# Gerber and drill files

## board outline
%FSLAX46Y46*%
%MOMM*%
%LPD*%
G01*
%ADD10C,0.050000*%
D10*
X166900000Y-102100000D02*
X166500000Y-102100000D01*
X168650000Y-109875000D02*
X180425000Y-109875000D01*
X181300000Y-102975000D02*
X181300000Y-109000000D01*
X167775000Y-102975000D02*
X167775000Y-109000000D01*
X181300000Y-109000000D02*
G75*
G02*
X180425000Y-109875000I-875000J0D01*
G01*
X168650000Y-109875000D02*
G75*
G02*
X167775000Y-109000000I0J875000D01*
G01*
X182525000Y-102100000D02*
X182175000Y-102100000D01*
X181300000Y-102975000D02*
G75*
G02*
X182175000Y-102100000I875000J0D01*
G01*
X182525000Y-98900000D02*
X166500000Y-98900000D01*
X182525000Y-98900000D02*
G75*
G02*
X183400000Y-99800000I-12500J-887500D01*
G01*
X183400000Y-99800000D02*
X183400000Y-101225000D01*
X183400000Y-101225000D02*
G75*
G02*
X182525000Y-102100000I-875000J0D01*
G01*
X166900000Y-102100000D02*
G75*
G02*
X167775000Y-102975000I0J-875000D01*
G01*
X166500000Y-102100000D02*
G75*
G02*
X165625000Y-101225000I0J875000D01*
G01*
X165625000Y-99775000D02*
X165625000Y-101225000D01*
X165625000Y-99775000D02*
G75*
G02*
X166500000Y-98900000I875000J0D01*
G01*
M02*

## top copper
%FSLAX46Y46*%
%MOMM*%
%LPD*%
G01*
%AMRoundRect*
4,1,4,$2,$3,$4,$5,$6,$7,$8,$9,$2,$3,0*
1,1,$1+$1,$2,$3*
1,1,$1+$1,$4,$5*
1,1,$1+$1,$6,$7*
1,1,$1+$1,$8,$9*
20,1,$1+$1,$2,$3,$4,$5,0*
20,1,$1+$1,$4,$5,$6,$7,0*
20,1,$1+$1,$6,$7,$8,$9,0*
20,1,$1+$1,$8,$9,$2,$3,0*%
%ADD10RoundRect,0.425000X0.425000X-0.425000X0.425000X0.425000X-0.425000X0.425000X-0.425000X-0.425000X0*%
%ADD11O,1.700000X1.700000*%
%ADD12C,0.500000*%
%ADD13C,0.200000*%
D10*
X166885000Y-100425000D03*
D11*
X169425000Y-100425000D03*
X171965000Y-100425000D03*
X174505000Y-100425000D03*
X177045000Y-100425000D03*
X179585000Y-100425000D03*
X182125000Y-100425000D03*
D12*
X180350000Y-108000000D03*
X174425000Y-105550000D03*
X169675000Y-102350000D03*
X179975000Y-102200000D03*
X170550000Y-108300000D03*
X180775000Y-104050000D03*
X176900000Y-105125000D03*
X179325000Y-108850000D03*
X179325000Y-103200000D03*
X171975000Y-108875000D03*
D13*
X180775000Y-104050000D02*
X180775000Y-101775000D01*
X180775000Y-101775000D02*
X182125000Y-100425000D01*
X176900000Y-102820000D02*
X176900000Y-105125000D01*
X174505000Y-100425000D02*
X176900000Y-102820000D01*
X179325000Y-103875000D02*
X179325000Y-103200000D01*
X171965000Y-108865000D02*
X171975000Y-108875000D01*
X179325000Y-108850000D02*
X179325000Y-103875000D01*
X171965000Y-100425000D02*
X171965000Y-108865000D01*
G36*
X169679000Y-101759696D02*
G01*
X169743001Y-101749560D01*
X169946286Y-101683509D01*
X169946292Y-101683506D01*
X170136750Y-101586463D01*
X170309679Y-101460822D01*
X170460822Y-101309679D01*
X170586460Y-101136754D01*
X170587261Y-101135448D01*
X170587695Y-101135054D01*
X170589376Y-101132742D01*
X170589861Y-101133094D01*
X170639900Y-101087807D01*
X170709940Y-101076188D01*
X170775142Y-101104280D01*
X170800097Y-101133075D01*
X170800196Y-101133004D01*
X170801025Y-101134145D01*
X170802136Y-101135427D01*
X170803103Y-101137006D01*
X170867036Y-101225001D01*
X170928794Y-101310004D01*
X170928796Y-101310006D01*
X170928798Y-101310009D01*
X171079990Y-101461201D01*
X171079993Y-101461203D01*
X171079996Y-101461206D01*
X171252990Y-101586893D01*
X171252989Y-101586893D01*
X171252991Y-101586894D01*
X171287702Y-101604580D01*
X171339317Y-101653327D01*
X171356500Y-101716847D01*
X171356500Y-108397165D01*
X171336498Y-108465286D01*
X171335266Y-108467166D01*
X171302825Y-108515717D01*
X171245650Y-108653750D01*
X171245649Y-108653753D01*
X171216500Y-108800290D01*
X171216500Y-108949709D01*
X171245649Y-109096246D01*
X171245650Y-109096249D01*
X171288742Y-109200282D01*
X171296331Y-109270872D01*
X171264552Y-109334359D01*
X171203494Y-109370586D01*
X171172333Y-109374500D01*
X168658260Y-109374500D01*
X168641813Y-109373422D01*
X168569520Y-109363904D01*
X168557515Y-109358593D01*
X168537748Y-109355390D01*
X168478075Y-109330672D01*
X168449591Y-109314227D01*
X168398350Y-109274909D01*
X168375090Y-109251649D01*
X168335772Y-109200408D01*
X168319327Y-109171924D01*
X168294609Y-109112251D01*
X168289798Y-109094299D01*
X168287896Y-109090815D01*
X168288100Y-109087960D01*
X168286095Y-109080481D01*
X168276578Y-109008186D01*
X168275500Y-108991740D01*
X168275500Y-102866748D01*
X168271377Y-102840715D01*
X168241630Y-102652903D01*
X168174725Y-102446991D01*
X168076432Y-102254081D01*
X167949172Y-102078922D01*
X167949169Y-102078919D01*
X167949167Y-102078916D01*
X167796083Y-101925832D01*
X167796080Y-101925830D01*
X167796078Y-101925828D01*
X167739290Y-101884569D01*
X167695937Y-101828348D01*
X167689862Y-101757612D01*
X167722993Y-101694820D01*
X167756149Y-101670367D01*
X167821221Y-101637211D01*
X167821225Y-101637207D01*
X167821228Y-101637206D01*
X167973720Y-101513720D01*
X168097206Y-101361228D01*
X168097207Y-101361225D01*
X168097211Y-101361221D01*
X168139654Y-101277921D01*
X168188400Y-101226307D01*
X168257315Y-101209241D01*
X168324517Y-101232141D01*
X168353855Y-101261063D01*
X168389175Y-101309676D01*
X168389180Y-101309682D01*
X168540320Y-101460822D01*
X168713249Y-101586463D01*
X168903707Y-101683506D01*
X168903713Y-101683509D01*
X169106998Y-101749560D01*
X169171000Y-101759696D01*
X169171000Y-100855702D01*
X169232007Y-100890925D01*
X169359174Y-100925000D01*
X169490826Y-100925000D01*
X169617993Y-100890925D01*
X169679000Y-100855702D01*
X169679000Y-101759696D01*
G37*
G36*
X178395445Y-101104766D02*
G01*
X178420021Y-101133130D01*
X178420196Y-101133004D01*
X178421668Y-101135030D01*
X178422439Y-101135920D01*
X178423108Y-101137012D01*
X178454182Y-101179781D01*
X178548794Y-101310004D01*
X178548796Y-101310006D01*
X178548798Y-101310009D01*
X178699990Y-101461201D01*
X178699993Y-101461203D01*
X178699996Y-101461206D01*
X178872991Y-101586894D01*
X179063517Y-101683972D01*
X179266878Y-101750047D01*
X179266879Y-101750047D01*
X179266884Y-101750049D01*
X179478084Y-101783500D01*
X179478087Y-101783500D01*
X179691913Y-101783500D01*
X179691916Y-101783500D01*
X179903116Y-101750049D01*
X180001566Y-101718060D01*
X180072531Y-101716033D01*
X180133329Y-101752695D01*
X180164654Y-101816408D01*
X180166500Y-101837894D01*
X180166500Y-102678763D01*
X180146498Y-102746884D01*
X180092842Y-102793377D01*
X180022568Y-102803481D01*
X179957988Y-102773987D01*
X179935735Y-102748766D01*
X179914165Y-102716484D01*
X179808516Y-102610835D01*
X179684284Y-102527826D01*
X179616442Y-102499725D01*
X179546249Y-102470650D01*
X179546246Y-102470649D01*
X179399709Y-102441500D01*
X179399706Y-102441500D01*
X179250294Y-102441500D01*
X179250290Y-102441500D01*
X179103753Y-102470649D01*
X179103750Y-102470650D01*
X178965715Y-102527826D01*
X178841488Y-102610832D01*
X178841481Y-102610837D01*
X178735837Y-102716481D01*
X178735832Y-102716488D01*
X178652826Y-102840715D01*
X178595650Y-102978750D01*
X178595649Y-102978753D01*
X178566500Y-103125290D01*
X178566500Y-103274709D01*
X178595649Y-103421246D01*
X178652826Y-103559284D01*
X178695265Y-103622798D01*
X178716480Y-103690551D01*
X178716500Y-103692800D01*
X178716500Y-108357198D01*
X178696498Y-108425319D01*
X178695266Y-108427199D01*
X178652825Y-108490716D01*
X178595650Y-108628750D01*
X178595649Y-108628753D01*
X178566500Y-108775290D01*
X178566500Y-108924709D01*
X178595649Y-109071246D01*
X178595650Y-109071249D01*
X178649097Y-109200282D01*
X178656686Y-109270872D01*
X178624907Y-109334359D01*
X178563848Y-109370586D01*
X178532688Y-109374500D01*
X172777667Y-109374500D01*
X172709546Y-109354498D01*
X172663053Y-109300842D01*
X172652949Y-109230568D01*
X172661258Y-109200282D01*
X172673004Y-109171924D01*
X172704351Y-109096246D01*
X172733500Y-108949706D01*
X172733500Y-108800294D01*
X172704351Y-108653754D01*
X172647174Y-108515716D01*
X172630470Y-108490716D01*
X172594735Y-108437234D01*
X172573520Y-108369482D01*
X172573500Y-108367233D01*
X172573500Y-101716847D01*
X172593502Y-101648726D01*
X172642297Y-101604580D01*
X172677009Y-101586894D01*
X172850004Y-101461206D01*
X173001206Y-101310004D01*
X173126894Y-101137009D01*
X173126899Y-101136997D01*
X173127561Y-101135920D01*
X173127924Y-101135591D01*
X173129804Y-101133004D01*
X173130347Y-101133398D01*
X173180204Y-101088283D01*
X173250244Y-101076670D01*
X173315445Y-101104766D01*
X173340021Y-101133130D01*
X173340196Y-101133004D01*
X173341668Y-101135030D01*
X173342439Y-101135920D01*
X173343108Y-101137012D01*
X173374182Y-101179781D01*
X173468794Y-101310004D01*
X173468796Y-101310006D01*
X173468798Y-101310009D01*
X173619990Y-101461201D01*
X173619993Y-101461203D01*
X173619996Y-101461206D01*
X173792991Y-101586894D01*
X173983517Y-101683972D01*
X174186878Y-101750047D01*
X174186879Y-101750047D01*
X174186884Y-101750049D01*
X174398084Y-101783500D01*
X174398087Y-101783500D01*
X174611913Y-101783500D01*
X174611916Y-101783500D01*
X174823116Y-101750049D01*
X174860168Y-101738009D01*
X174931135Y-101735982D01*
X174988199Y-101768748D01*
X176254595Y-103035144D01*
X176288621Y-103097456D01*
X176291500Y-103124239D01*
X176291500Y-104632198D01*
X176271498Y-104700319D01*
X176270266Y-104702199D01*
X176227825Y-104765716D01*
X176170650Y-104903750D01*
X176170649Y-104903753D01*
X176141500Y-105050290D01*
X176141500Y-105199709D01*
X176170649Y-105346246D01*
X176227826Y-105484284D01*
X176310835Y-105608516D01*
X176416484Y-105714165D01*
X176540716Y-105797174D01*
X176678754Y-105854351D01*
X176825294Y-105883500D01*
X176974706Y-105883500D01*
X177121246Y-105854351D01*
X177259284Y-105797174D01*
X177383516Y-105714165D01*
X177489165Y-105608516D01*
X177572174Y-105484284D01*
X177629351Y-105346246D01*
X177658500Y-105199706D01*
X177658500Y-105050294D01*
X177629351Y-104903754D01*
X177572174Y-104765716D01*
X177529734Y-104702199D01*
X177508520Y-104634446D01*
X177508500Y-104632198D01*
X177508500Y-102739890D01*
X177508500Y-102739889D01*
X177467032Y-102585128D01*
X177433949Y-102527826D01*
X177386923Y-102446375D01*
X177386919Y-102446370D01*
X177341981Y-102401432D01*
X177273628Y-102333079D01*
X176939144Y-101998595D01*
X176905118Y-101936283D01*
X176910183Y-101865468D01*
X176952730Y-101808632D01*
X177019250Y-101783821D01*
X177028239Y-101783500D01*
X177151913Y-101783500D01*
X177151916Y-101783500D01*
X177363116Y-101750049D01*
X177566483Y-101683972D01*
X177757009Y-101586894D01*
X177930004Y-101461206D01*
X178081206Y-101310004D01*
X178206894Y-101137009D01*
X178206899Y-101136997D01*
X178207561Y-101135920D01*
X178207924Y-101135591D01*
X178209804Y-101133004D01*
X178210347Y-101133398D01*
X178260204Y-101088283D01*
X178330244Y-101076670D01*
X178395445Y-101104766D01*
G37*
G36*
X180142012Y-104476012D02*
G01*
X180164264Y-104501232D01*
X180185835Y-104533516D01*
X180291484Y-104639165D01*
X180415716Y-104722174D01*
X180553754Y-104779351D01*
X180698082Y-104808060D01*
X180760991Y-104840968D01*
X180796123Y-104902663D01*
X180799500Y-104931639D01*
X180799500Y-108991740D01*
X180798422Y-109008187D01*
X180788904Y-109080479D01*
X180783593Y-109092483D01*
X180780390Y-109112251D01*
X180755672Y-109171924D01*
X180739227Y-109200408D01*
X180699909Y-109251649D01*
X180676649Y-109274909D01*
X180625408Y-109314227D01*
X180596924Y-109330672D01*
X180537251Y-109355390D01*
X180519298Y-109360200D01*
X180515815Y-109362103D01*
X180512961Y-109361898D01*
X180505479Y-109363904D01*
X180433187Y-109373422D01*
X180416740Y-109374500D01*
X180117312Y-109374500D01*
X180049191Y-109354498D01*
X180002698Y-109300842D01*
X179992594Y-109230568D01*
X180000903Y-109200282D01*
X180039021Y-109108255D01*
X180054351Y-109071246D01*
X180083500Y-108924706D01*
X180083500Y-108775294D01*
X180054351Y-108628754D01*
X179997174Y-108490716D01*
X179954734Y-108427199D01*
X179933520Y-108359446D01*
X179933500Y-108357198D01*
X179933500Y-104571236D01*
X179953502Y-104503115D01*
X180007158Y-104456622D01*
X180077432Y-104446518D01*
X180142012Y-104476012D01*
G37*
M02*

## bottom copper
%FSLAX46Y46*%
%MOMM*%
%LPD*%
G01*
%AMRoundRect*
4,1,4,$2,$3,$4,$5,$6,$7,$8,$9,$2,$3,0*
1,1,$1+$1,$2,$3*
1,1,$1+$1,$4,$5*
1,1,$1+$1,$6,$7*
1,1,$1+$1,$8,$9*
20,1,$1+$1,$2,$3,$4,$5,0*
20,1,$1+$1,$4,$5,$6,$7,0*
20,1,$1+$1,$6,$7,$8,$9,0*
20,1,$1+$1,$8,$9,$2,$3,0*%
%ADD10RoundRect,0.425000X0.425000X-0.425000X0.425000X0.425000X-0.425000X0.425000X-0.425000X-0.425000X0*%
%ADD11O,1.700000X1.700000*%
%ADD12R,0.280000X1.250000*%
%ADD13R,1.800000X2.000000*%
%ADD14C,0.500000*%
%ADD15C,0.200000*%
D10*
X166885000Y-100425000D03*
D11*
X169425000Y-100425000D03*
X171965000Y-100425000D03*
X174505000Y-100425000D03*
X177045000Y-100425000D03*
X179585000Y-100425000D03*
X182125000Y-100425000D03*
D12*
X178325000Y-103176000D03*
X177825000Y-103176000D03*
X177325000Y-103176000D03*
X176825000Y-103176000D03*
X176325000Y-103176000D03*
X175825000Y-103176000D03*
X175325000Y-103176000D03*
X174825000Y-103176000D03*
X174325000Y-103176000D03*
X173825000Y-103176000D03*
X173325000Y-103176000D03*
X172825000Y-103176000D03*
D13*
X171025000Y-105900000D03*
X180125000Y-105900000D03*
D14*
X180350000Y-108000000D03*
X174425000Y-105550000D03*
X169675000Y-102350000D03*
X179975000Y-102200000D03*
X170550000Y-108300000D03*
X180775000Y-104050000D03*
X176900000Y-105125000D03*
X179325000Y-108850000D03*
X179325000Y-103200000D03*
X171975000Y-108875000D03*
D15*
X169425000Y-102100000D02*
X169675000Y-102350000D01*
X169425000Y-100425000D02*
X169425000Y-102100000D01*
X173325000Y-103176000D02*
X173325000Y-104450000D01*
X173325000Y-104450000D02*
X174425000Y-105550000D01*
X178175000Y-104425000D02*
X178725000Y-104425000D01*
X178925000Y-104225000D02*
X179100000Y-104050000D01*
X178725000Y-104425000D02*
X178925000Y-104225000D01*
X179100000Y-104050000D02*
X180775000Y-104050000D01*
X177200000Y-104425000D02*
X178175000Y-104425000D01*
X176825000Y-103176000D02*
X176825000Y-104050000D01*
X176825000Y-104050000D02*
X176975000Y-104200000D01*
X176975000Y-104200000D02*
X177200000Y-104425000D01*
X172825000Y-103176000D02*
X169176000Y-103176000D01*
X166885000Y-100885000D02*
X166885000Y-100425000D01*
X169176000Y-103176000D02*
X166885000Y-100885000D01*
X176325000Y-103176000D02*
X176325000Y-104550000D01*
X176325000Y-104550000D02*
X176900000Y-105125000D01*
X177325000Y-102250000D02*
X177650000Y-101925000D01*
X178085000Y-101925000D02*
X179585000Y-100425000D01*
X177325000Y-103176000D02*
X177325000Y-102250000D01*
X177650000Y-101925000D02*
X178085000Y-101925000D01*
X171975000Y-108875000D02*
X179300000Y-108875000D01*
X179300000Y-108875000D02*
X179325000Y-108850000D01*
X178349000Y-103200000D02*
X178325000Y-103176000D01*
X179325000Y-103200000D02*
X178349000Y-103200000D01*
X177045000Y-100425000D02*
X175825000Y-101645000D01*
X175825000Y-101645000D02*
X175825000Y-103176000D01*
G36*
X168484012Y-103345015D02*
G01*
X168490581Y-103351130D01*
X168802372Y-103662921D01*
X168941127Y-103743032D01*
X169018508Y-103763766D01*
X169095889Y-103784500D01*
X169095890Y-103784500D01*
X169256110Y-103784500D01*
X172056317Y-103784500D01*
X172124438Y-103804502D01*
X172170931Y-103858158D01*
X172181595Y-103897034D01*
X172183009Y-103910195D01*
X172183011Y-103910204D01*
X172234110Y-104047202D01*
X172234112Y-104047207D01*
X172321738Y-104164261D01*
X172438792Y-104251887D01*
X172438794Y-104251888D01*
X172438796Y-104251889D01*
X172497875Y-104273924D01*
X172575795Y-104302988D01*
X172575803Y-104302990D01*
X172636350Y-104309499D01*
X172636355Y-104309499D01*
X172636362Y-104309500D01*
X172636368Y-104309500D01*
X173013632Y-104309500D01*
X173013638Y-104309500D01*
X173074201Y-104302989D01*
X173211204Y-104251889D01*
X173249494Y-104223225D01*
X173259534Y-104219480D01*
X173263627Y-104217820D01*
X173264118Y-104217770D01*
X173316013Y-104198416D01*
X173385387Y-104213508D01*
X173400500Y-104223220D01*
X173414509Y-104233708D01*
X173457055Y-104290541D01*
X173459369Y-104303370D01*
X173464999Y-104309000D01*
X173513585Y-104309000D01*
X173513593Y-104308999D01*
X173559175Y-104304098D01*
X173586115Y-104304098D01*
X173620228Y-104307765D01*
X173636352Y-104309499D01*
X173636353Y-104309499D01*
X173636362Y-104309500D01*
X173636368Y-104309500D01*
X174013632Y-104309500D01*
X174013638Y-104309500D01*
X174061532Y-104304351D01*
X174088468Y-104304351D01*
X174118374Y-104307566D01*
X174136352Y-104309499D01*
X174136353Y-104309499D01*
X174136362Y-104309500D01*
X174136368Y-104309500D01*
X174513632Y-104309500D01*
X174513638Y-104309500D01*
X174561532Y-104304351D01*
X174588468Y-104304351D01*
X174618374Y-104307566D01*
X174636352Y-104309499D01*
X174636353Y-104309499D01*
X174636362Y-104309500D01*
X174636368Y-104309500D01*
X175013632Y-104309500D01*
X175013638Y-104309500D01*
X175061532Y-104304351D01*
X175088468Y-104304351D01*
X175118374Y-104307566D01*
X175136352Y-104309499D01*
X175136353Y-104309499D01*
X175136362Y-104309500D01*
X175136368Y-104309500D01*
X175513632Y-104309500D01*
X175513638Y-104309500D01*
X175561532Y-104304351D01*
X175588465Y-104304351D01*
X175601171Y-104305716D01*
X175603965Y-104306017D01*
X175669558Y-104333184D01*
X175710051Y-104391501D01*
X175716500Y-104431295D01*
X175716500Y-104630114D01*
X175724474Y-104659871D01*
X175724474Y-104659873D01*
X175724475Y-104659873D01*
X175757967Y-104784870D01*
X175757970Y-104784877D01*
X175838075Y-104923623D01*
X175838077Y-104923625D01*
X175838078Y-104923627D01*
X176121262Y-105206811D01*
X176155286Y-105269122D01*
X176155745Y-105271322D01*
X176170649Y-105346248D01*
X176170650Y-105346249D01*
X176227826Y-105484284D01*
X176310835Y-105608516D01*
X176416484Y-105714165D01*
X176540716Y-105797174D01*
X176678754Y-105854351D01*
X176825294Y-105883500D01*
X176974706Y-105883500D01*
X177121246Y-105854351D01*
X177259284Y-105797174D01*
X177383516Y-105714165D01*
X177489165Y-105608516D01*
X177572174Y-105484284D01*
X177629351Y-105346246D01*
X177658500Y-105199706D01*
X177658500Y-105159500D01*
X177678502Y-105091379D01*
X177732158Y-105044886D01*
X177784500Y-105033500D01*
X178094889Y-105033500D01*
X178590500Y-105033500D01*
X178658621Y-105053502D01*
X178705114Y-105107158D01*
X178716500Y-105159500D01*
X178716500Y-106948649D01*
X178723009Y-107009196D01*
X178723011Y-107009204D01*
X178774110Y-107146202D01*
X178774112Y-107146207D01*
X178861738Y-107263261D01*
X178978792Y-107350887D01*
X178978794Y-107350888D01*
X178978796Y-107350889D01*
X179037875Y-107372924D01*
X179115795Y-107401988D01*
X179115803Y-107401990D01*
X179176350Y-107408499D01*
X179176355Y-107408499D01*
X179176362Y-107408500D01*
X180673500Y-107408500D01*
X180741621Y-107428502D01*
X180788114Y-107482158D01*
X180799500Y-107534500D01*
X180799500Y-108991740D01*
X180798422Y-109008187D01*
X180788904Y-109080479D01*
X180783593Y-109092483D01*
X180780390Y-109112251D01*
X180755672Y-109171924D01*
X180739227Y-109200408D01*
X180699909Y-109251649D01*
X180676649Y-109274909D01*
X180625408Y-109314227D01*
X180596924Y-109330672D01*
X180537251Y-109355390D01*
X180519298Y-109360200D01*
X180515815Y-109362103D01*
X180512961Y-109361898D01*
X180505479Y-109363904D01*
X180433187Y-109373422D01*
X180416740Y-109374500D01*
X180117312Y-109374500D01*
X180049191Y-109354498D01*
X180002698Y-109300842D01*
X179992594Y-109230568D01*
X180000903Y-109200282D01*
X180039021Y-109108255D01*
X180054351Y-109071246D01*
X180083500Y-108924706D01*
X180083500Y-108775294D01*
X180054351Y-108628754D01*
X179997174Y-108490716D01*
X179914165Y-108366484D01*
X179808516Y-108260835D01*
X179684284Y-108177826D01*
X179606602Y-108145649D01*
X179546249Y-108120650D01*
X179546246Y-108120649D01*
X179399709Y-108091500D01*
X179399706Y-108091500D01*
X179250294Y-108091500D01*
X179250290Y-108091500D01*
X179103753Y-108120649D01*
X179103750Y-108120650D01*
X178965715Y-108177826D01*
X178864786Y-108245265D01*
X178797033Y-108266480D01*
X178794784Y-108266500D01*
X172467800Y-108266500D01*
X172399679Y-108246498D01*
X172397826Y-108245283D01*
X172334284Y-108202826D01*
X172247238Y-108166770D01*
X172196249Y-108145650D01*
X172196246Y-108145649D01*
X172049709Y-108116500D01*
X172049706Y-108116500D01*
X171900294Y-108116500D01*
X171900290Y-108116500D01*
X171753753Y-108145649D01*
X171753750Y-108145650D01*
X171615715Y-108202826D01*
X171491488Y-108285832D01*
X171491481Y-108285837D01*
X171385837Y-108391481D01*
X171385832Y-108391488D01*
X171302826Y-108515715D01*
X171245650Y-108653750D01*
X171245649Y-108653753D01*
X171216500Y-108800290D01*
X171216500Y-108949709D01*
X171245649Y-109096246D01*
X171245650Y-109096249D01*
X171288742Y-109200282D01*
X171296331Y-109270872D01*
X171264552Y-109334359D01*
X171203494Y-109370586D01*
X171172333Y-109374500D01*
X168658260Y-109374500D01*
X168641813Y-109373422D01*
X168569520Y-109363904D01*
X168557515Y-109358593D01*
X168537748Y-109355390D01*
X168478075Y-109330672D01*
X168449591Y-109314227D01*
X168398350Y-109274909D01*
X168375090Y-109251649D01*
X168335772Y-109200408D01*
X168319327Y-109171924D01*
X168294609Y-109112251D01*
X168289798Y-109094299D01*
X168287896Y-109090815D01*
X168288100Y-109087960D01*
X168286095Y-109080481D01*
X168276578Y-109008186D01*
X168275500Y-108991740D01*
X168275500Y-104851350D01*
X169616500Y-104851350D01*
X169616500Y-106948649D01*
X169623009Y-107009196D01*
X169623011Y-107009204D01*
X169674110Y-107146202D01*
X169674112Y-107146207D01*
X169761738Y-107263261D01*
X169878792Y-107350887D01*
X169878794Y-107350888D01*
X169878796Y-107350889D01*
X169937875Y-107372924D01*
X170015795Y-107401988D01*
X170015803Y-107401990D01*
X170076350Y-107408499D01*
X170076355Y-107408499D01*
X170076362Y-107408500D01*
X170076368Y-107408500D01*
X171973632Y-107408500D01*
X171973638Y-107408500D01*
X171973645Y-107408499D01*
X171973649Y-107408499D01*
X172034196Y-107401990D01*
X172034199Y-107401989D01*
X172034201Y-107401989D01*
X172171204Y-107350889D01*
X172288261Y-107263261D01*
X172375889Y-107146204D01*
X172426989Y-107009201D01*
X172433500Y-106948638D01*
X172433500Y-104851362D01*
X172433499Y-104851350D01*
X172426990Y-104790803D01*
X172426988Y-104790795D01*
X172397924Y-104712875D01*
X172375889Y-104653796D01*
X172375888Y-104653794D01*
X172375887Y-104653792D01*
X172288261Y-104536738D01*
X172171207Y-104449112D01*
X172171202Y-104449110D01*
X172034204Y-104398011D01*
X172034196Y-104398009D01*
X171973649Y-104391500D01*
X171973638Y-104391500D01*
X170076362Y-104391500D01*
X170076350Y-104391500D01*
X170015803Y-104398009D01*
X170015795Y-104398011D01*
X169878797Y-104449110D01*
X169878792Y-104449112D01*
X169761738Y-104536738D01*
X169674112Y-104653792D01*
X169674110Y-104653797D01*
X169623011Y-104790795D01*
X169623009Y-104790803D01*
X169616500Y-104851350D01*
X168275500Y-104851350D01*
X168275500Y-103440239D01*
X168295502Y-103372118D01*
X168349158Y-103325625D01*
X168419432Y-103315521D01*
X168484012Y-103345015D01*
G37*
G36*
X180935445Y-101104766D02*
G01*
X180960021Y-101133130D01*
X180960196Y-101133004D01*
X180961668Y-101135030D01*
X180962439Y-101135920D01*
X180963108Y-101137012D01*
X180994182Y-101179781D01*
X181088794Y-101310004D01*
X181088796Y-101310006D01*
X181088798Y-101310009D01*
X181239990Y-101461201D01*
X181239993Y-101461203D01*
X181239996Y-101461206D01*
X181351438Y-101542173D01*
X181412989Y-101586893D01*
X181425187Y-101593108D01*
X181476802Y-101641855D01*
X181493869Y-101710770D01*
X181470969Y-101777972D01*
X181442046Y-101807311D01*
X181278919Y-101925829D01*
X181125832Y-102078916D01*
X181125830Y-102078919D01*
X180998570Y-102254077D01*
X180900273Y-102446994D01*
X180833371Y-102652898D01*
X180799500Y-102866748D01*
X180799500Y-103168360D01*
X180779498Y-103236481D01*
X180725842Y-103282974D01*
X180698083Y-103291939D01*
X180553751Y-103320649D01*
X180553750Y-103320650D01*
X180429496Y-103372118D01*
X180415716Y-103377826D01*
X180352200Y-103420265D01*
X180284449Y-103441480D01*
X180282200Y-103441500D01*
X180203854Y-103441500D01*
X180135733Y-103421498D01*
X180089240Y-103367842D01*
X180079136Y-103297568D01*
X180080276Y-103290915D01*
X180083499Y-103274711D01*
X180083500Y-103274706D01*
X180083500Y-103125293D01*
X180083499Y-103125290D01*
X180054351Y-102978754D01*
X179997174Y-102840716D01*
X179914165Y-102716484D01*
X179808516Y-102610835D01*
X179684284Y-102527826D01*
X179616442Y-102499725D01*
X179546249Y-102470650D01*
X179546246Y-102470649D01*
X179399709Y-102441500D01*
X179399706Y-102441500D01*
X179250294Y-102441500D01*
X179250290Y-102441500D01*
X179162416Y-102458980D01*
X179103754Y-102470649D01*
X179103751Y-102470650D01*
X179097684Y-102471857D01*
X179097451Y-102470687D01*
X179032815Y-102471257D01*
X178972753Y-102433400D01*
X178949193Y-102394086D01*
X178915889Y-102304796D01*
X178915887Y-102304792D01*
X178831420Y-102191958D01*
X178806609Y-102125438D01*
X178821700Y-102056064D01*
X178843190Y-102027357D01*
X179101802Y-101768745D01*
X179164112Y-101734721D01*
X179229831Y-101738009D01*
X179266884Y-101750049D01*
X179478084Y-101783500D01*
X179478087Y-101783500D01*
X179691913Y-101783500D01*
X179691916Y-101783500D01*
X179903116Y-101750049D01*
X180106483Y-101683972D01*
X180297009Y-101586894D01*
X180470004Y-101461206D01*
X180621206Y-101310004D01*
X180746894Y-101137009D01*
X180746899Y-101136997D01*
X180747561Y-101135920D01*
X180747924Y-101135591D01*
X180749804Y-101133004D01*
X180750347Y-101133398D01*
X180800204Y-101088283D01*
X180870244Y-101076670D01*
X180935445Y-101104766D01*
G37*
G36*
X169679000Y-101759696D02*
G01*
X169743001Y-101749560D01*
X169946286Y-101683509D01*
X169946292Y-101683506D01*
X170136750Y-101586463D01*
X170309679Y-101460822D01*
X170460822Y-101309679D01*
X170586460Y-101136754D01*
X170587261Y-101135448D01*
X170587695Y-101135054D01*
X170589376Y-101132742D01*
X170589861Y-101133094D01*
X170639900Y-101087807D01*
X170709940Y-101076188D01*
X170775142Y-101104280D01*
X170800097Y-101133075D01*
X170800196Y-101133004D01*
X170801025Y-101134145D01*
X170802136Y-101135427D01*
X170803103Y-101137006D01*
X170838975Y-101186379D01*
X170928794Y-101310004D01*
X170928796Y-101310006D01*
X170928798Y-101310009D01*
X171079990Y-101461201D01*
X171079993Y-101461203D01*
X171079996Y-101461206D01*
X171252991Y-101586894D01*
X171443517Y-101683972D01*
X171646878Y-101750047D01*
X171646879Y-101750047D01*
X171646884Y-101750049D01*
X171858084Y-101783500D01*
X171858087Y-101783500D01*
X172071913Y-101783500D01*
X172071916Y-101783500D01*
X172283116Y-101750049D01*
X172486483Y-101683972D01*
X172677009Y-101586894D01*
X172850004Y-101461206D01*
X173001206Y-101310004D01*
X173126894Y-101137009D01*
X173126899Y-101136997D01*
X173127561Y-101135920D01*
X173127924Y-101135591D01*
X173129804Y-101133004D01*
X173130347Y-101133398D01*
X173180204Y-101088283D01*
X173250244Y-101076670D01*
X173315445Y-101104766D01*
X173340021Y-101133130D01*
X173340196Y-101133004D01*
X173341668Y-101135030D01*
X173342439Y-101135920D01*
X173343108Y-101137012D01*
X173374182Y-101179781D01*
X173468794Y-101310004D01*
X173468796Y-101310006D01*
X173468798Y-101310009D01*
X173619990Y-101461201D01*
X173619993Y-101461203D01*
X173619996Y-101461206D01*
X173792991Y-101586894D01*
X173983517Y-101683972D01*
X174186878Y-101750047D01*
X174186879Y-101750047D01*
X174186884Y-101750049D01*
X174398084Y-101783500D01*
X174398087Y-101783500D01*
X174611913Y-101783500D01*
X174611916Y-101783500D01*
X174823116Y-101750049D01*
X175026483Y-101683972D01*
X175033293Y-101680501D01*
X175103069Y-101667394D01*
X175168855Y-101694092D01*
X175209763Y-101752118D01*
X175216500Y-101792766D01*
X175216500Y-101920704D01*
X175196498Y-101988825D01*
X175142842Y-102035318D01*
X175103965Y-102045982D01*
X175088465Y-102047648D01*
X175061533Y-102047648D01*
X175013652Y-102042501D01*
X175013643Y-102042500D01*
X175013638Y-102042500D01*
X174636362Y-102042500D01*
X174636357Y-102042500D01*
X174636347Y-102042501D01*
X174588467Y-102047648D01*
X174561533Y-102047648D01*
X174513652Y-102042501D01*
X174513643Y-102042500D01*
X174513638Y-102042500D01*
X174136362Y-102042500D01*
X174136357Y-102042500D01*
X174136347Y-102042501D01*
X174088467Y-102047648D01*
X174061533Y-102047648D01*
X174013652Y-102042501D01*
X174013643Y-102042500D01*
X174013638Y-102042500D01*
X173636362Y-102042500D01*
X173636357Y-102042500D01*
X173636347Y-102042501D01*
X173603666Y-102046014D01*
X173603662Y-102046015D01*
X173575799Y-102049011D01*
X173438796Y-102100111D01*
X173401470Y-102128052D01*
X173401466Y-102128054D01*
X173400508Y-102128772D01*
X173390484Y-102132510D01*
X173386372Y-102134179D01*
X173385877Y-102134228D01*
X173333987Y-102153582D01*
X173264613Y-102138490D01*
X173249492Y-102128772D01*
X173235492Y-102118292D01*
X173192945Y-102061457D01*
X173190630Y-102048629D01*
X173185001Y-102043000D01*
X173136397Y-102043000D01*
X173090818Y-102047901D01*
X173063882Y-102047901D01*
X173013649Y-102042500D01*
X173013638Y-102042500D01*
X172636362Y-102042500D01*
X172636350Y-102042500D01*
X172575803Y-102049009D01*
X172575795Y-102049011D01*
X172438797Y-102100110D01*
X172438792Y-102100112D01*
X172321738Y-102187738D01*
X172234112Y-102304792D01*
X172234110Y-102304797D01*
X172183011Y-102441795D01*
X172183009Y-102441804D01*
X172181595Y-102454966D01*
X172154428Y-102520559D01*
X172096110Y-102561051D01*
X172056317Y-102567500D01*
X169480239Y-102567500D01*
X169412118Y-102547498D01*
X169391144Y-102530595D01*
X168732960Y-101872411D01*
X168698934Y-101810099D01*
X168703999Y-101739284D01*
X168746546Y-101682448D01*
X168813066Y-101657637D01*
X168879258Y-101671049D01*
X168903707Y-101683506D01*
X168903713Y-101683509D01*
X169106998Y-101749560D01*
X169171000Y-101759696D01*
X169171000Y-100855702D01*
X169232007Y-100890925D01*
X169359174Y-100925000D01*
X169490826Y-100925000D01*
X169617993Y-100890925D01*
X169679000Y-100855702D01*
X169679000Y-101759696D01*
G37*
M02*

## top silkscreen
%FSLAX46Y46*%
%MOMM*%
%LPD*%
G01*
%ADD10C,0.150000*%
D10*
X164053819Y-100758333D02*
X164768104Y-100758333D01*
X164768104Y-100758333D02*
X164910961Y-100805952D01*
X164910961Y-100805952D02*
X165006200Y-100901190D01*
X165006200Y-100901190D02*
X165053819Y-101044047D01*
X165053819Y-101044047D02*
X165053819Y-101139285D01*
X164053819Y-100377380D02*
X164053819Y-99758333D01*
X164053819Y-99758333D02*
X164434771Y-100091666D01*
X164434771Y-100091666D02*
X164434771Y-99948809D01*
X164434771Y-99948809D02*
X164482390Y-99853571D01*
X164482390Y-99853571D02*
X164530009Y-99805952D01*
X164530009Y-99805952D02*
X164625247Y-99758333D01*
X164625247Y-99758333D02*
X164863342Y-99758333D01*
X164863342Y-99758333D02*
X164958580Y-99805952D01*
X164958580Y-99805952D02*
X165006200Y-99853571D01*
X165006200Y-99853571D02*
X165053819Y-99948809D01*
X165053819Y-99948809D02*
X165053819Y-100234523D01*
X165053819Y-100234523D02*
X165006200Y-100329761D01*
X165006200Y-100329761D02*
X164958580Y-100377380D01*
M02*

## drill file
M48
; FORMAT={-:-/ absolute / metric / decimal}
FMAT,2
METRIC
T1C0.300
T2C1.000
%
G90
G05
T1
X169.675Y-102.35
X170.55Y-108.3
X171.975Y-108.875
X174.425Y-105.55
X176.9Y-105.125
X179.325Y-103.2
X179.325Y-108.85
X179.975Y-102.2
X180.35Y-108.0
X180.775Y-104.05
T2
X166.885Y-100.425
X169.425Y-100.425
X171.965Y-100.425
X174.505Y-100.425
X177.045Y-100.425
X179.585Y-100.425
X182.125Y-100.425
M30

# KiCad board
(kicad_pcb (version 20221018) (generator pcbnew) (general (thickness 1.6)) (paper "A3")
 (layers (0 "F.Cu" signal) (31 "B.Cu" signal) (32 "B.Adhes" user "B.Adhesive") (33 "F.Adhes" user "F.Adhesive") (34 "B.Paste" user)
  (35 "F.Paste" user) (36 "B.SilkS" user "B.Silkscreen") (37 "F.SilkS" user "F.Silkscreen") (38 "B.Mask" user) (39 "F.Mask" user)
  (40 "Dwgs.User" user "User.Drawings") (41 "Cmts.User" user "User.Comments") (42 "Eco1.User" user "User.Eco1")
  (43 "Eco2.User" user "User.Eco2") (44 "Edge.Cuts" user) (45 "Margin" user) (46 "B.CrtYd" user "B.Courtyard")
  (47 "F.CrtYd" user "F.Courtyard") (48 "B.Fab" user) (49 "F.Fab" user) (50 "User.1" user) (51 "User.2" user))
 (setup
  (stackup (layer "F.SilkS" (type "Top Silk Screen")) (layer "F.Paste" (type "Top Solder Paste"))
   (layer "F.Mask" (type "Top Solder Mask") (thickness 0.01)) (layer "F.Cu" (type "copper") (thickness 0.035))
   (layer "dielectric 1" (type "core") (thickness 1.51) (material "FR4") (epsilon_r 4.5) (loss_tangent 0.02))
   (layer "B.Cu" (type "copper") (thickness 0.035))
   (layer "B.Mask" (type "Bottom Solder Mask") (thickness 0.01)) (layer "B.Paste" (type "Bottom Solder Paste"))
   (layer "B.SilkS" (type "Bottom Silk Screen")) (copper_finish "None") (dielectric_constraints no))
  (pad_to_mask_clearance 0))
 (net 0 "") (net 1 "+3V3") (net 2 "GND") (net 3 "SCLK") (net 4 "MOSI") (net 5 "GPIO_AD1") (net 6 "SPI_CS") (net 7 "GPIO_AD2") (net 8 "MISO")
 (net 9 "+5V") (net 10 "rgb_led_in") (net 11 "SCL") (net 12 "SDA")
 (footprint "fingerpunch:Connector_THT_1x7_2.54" (layer "F.Cu") (at 170.695 100.425 90)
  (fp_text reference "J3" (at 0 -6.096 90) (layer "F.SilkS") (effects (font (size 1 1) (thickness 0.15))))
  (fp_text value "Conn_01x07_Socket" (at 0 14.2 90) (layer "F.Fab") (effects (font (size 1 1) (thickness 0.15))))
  (pad "1" thru_hole roundrect (at 0 -3.81 90) (size 1.7 1.7) (drill 1) (layers "*.Cu" "*.Mask") (roundrect_rratio 0.25) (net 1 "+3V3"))
  (pad "2" thru_hole oval (at 0 -1.27 90) (size 1.7 1.7) (drill 1) (layers "*.Cu" "*.Mask") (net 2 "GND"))
  (pad "3" thru_hole oval (at 0 1.27 90) (size 1.7 1.7) (drill 1) (layers "*.Cu" "*.Mask") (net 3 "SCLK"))
  (pad "4" thru_hole oval (at 0 3.81 90) (size 1.7 1.7) (drill 1) (layers "*.Cu" "*.Mask") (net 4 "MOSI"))
  (pad "5" thru_hole oval (at 0 6.35 90) (size 1.7 1.7) (drill 1) (layers "*.Cu" "*.Mask") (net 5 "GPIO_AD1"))
  (pad "6" thru_hole oval (at 0 8.89 90) (size 1.7 1.7) (drill 1) (layers "*.Cu" "*.Mask") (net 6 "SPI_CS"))
  (pad "7" thru_hole oval (at 0 11.43 90) (size 1.7 1.7) (drill 1) (layers "*.Cu" "*.Mask") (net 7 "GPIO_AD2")))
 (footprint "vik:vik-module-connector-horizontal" (layer "B.Cu") (at 175.575 105.214 180)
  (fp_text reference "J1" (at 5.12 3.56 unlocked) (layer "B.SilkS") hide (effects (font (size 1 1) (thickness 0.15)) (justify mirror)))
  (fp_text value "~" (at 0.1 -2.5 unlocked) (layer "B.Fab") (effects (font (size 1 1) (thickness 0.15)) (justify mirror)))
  (pad "1" smd rect (at -2.75 2.038 180) (size 0.28 1.25) (layers "B.Cu" "B.Paste" "B.Mask") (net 3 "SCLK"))
  (pad "2" smd rect (at -2.25 2.038 180) (size 0.28 1.25) (layers "B.Cu" "B.Paste" "B.Mask") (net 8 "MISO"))
  (pad "3" smd rect (at -1.75 2.038 180) (size 0.28 1.25) (layers "B.Cu" "B.Paste" "B.Mask") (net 6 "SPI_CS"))
  (pad "4" smd rect (at -1.25 2.038 180) (size 0.28 1.25) (layers "B.Cu" "B.Paste" "B.Mask") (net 7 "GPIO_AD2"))
  (pad "5" smd rect (at -0.75 2.038 180) (size 0.28 1.25) (layers "B.Cu" "B.Paste" "B.Mask") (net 4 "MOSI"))
  (pad "6" smd rect (at -0.25 2.038 180) (size 0.28 1.25) (layers "B.Cu" "B.Paste" "B.Mask") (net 5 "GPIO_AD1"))
  (pad "7" smd rect (at 0.25 2.038 180) (size 0.28 1.25) (layers "B.Cu" "B.Paste" "B.Mask") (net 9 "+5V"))
  (pad "8" smd rect (at 0.75 2.038 180) (size 0.28 1.25) (layers "B.Cu" "B.Paste" "B.Mask") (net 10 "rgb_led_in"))
  (pad "9" smd rect (at 1.25 2.038 180) (size 0.28 1.25) (layers "B.Cu" "B.Paste" "B.Mask") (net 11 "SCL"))
  (pad "10" smd rect (at 1.75 2.038 180) (size 0.28 1.25) (layers "B.Cu" "B.Paste" "B.Mask") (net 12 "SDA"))
  (pad "11" smd rect (at 2.25 2.038 180) (size 0.28 1.25) (layers "B.Cu" "B.Paste" "B.Mask") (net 2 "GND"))
  (pad "12" smd rect (at 2.75 2.038 180) (size 0.28 1.25) (layers "B.Cu" "B.Paste" "B.Mask") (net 1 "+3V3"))
  (pad "13" smd rect (at 4.55 -0.686 180) (size 1.8 2) (layers "B.Cu" "B.Paste" "B.Mask"))
  (pad "14" smd rect (at -4.55 -0.686 180) (size 1.8 2) (layers "B.Cu" "B.Paste" "B.Mask")))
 (gr_line (start 166.9 102.1) (end 166.5 102.1) (stroke (width 0.05) (type solid)) (layer "Edge.Cuts"))
 (gr_line (start 168.65 109.875) (end 180.425 109.875) (stroke (width 0.05) (type solid)) (layer "Edge.Cuts"))
 (gr_line (start 181.3 102.975) (end 181.3 109) (stroke (width 0.05) (type solid)) (layer "Edge.Cuts"))
 (gr_line (start 167.775 102.975) (end 167.775 109) (stroke (width 0.05) (type solid)) (layer "Edge.Cuts"))
 (gr_arc (start 181.3 109) (mid 181.043718 109.618718) (end 180.425 109.875) (stroke (width 0.05) (type solid)) (layer "Edge.Cuts"))
 (gr_arc (start 168.65 109.875) (mid 168.031282 109.618718) (end 167.775 109) (stroke (width 0.05) (type solid)) (layer "Edge.Cuts"))
 (gr_line (start 182.525 102.1) (end 182.175 102.1) (stroke (width 0.05) (type solid)) (layer "Edge.Cuts"))
 (gr_arc (start 181.3 102.975) (mid 181.556282 102.356282) (end 182.175 102.1) (stroke (width 0.05) (type solid)) (layer "Edge.Cuts"))
 (gr_line (start 182.525 98.9) (end 166.5 98.9) (stroke (width 0.05) (type solid)) (layer "Edge.Cuts"))
 (gr_arc (start 182.525 98.9) (mid 183.148896 99.168782) (end 183.4 99.8) (stroke (width 0.05) (type solid)) (layer "Edge.Cuts"))
 (gr_line (start 183.4 99.8) (end 183.4 101.225) (stroke (width 0.05) (type solid)) (layer "Edge.Cuts"))
 (gr_arc (start 183.4 101.225) (mid 183.143718 101.843718) (end 182.525 102.1) (stroke (width 0.05) (type solid)) (layer "Edge.Cuts"))
 (gr_arc (start 166.9 102.1) (mid 167.518718 102.356282) (end 167.775 102.975) (stroke (width 0.05) (type solid)) (layer "Edge.Cuts"))
 (gr_arc (start 166.5 102.1) (mid 165.881282 101.843718) (end 165.625 101.225) (stroke (width 0.05) (type solid)) (layer "Edge.Cuts"))
 (gr_line (start 165.625 99.775) (end 165.625 101.225) (stroke (width 0.05) (type solid)) (layer "Edge.Cuts"))
 (gr_arc (start 165.625 99.775) (mid 165.881282 99.156282) (end 166.5 98.9) (stroke (width 0.05) (type solid)) (layer "Edge.Cuts"))
 (via (at 180.35 108) (size 0.5) (drill 0.3) (layers "F.Cu" "B.Cu") (free) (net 2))
 (via (at 174.425 105.55) (size 0.5) (drill 0.3) (layers "F.Cu" "B.Cu") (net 2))
 (via (at 169.675 102.35) (size 0.5) (drill 0.3) (layers "F.Cu" "B.Cu") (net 2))
 (via (at 179.975 102.2) (size 0.5) (drill 0.3) (layers "F.Cu" "B.Cu") (free) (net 2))
 (via (at 170.55 108.3) (size 0.5) (drill 0.3) (layers "F.Cu" "B.Cu") (free) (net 2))
 (segment (start 169.425 102.1) (end 169.675 102.35) (width 0.2) (layer "B.Cu") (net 2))
 (segment (start 169.425 100.425) (end 169.425 102.1) (width 0.2) (layer "B.Cu") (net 2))
 (segment (start 173.325 103.176) (end 173.325 104.45) (width 0.2) (layer "B.Cu") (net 2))
 (segment (start 173.325 104.45) (end 174.425 105.55) (width 0.2) (layer "B.Cu") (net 2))
 (segment (start 180.775 104.05) (end 180.775 101.775) (width 0.2) (layer "F.Cu") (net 7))
 (segment (start 180.775 101.775) (end 182.125 100.425) (width 0.2) (layer "F.Cu") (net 7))
 (via (at 180.775 104.05) (size 0.5) (drill 0.3) (layers "F.Cu" "B.Cu") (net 7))
 (segment (start 178.175 104.425) (end 178.725 104.425) (width 0.2) (layer "B.Cu") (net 7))
 (segment (start 178.925 104.225) (end 179.1 104.05) (width 0.2) (layer "B.Cu") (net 7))
 (segment (start 178.725 104.425) (end 178.925 104.225) (width 0.2) (layer "B.Cu") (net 7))
 (segment (start 179.1 104.05) (end 180.775 104.05) (width 0.2) (layer "B.Cu") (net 7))
 (segment (start 177.2 104.425) (end 178.175 104.425) (width 0.2) (layer "B.Cu") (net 7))
 (segment (start 176.825 103.176) (end 176.825 104.05) (width 0.2) (layer "B.Cu") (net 7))
 (segment (start 176.825 104.05) (end 176.975 104.2) (width 0.2) (layer "B.Cu") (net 7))
 (segment (start 176.975 104.2) (end 177.2 104.425) (width 0.2) (layer "B.Cu") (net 7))
 (segment (start 172.825 103.176) (end 169.176 103.176) (width 0.2) (layer "B.Cu") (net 1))
 (segment (start 166.885 100.885) (end 166.885 100.425) (width 0.2) (layer "B.Cu") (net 1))
 (segment (start 169.176 103.176) (end 166.885 100.885) (width 0.2) (layer "B.Cu") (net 1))
 (segment (start 176.9 102.82) (end 176.9 105.125) (width 0.2) (layer "F.Cu") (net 4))
 (segment (start 174.505 100.425) (end 176.9 102.82) (width 0.2) (layer "F.Cu") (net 4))
 (via (at 176.9 105.125) (size 0.5) (drill 0.3) (layers "F.Cu" "B.Cu") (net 4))
 (segment (start 176.325 103.176) (end 176.325 104.55) (width 0.2) (layer "B.Cu") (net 4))
 (segment (start 176.325 104.55) (end 176.9 105.125) (width 0.2) (layer "B.Cu") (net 4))
 (segment (start 177.325 102.25) (end 177.65 101.925) (width 0.2) (layer "B.Cu") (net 6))
 (segment (start 178.085 101.925) (end 179.585 100.425) (width 0.2) (layer "B.Cu") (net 6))
 (segment (start 177.325 103.176) (end 177.325 102.25) (width 0.2) (layer "B.Cu") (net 6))
 (segment (start 177.65 101.925) (end 178.085 101.925) (width 0.2) (layer "B.Cu") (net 6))
 (segment (start 179.325 103.875) (end 179.325 103.2) (width 0.2) (layer "F.Cu") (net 3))
 (segment (start 171.965 108.865) (end 171.975 108.875) (width 0.2) (layer "F.Cu") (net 3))
 (segment (start 179.325 108.85) (end 179.325 103.875) (width 0.2) (layer "F.Cu") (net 3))
 (segment (start 171.965 100.425) (end 171.965 108.865) (width 0.2) (layer "F.Cu") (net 3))
 (via (at 179.325 108.85) (size 0.5) (drill 0.3) (layers "F.Cu" "B.Cu") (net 3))
 (via (at 179.325 103.2) (size 0.5) (drill 0.3) (layers "F.Cu" "B.Cu") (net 3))
 (via (at 171.975 108.875) (size 0.5) (drill 0.3) (layers "F.Cu" "B.Cu") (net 3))
 (segment (start 171.975 108.875) (end 179.3 108.875) (width 0.2) (layer "B.Cu") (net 3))
 (segment (start 179.3 108.875) (end 179.325 108.85) (width 0.2) (layer "B.Cu") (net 3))
 (segment (start 178.349 103.2) (end 178.325 103.176) (width 0.2) (layer "B.Cu") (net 3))
 (segment (start 179.325 103.2) (end 178.349 103.2) (width 0.2) (layer "B.Cu") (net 3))
 (segment (start 177.045 100.425) (end 175.825 101.645) (width 0.2) (layer "B.Cu") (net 5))
 (segment (start 175.825 101.645) (end 175.825 103.176) (width 0.2) (layer "B.Cu") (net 5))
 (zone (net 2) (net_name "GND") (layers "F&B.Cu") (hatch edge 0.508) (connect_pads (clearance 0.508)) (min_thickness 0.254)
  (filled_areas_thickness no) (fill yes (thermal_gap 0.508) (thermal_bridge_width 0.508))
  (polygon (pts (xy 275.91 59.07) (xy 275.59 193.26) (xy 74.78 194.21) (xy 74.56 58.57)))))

